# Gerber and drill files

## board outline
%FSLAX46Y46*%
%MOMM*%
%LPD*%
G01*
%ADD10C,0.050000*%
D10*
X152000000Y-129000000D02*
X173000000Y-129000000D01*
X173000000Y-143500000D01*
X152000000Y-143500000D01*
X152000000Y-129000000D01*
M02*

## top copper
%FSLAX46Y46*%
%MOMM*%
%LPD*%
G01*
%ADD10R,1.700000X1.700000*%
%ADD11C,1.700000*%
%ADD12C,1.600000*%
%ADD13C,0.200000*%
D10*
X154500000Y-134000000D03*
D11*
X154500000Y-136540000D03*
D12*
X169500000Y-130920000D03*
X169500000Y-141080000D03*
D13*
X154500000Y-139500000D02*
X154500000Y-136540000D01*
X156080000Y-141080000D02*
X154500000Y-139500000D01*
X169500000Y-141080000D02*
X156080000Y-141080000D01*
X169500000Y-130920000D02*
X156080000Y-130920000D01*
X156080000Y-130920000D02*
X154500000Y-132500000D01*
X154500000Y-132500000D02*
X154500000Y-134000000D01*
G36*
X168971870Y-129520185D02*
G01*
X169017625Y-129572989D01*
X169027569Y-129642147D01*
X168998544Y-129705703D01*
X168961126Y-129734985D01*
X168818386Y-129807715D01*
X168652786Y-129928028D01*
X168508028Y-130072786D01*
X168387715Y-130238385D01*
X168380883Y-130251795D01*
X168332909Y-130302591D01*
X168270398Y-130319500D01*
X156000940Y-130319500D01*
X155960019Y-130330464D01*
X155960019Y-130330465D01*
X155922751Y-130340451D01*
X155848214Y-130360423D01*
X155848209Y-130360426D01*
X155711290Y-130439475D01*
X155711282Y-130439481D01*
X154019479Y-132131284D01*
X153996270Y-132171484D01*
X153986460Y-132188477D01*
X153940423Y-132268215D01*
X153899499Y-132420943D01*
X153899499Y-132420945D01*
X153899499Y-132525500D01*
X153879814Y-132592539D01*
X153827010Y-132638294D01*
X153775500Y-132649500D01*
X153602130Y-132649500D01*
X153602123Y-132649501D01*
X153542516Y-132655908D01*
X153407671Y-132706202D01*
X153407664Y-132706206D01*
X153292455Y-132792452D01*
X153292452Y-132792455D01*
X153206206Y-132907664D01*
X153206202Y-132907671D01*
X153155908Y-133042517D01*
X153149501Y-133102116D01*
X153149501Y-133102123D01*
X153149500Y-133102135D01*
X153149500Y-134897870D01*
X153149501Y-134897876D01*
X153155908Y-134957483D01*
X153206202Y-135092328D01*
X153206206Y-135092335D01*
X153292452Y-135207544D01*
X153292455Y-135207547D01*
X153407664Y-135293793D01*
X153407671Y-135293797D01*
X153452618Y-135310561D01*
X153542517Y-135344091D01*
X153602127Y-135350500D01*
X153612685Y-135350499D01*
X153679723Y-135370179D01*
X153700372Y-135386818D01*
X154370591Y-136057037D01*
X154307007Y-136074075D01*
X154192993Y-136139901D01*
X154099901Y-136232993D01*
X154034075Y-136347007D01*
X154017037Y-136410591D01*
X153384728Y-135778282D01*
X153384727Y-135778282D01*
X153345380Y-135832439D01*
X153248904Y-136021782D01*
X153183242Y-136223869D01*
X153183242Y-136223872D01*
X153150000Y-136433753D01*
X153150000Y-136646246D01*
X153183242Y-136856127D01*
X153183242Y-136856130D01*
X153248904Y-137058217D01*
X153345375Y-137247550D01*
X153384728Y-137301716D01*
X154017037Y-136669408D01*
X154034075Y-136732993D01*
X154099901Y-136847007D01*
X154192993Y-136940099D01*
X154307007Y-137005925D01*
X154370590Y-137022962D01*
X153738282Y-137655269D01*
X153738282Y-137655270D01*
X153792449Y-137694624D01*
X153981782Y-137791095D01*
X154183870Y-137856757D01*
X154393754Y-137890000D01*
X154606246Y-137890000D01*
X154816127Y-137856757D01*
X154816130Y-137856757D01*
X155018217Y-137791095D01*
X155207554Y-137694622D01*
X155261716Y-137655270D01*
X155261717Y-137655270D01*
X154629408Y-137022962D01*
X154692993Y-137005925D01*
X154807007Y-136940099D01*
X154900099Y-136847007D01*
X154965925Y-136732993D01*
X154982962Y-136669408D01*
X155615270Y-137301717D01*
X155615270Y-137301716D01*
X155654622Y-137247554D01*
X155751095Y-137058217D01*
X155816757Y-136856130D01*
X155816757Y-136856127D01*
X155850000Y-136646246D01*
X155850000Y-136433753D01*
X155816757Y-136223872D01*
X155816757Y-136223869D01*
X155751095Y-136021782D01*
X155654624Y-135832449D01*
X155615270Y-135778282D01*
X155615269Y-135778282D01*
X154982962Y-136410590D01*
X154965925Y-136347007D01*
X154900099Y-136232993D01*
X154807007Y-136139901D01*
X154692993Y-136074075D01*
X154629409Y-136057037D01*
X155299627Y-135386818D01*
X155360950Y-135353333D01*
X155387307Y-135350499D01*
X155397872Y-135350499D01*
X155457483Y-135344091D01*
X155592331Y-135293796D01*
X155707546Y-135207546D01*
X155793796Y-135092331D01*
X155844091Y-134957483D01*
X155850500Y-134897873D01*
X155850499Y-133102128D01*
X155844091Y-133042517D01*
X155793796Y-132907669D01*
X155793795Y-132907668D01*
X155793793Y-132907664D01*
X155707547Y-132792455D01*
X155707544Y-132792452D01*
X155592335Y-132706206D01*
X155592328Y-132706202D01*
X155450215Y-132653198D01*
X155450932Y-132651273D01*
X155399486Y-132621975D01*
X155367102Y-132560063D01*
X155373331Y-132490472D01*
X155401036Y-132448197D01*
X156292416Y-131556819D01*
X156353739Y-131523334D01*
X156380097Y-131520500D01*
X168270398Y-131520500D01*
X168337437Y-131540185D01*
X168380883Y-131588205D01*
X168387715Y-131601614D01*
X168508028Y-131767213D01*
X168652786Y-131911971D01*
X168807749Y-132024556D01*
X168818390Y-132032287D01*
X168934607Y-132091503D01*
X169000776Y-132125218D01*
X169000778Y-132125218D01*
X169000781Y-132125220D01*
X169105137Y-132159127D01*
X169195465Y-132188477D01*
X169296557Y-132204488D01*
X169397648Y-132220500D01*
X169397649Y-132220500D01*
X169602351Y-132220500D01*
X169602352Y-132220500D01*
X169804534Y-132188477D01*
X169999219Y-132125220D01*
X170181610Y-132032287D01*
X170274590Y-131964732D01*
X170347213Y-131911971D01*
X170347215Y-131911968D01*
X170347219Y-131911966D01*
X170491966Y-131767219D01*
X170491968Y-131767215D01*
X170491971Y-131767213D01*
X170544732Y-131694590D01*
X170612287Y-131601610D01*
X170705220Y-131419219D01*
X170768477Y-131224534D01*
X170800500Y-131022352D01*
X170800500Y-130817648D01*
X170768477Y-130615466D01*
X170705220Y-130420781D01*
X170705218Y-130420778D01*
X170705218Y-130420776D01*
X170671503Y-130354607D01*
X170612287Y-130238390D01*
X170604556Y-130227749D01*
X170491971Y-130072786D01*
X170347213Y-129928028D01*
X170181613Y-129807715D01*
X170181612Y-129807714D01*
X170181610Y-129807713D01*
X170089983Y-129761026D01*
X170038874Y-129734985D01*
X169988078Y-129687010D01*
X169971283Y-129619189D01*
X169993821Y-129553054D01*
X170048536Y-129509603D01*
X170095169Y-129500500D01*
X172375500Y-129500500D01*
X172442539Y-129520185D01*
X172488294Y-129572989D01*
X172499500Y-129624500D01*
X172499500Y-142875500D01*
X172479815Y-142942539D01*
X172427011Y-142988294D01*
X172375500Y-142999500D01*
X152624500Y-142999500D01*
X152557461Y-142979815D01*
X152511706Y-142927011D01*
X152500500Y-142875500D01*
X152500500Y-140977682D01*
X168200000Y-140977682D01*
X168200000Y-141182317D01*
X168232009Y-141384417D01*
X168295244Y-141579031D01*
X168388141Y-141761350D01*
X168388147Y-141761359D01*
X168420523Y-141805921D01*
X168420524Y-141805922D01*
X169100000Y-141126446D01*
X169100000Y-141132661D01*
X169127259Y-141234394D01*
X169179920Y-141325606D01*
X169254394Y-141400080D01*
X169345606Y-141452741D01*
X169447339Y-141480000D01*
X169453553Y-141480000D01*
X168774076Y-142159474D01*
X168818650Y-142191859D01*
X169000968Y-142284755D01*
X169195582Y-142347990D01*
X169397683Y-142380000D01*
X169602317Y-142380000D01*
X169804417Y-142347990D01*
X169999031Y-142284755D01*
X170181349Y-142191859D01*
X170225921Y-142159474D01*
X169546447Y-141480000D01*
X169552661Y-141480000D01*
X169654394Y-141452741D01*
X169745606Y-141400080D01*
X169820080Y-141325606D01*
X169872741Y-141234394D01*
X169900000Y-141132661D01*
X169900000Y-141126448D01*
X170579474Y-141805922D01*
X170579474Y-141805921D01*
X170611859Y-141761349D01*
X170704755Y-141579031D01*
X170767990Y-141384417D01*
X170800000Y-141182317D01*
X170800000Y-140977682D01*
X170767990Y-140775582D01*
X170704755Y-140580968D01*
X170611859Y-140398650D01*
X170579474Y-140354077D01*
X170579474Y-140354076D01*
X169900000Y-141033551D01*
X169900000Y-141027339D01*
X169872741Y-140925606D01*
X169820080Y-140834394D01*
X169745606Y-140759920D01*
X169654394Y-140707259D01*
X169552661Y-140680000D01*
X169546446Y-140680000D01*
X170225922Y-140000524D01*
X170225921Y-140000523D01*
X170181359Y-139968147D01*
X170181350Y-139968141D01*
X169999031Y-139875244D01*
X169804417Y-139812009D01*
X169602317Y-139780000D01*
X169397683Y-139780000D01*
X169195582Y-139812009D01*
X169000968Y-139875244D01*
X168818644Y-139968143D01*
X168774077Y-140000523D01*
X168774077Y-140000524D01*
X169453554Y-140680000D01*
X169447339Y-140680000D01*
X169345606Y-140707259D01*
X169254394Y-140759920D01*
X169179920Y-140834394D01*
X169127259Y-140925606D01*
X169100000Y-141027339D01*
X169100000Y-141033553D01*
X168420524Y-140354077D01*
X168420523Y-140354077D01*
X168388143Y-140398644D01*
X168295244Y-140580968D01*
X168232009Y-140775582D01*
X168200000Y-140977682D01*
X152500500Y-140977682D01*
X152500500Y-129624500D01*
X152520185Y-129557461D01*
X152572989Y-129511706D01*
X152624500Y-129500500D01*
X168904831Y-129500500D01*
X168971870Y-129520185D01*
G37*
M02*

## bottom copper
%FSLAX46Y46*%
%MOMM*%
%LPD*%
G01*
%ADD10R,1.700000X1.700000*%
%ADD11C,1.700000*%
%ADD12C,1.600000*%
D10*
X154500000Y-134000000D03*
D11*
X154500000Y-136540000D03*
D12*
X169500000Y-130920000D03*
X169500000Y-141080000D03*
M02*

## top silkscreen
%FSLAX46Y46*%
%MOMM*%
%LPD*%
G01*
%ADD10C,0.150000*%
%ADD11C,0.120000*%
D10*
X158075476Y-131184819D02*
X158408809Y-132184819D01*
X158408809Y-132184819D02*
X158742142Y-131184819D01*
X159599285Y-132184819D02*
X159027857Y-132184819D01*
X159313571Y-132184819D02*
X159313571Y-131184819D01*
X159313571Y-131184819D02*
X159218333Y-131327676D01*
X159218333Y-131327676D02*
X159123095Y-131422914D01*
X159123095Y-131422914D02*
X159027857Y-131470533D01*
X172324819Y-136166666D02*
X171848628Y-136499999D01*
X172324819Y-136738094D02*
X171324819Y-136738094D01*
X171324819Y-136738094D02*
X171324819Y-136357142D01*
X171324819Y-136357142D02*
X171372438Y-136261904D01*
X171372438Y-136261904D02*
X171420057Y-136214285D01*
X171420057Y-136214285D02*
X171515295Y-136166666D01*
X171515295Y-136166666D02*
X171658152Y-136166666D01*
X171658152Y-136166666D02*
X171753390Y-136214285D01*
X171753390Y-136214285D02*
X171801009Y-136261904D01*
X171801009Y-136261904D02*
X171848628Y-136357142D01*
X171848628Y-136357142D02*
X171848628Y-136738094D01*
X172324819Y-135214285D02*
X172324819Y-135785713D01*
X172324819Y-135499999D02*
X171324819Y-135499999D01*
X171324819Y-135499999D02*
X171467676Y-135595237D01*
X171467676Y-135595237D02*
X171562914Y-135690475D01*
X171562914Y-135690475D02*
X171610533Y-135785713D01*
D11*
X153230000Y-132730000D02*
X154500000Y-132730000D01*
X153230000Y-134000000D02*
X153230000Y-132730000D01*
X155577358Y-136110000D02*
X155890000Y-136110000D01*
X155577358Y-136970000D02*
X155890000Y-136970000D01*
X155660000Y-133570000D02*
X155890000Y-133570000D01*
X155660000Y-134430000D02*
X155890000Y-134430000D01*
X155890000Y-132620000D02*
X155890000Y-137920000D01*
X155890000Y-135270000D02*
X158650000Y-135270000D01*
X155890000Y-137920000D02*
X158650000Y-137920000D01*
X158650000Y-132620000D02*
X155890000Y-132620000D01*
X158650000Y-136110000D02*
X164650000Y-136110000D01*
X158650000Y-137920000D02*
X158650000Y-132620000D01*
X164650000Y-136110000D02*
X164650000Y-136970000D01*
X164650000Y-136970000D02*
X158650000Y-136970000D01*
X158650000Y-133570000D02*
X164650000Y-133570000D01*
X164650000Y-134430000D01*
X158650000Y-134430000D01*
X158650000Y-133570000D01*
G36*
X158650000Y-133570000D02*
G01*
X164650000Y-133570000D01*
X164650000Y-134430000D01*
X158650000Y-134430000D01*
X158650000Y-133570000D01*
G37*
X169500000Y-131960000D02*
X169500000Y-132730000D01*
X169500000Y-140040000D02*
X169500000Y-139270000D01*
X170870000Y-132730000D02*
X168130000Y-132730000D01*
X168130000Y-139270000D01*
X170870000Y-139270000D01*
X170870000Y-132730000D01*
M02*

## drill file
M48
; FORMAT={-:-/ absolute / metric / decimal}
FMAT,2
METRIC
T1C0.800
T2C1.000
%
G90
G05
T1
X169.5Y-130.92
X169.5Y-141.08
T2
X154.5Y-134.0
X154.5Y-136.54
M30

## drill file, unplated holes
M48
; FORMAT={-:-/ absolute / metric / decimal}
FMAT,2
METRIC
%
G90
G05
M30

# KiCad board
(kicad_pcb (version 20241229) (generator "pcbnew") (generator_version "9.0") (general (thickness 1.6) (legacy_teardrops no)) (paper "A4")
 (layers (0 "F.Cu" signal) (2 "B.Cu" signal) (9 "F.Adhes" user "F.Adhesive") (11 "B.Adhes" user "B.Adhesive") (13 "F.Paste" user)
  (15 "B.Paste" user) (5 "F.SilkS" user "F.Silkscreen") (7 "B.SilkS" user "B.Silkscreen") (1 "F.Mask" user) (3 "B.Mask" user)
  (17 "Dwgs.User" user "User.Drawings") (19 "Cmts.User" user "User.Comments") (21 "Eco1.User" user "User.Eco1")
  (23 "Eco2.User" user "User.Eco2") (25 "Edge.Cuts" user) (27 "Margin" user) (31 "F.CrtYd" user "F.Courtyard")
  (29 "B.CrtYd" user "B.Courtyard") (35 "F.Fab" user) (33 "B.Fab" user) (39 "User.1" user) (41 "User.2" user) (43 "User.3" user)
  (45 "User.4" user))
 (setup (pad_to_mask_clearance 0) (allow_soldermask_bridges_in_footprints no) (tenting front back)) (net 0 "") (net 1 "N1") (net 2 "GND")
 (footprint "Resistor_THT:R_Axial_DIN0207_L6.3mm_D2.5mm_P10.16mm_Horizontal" (layer "F.Cu") (at 169.5 130.92 -90)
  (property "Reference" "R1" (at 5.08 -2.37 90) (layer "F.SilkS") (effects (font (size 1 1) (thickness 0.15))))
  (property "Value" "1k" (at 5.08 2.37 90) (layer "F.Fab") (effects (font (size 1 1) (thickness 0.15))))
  (fp_line (start 1.04 0) (end 1.81 0) (stroke (width 0.12) (type solid)) (layer "F.SilkS"))
  (fp_line (start 9.12 0) (end 8.35 0) (stroke (width 0.12) (type solid)) (layer "F.SilkS"))
  (fp_rect (start 1.81 -1.37) (end 8.35 1.37) (stroke (width 0.12) (type solid)) (fill no) (layer "F.SilkS"))
  (pad "1" thru_hole circle (at 0 0 270) (size 1.6 1.6) (drill 0.8) (layers "*.Cu" "*.Mask") (remove_unused_layers no) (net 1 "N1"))
  (pad "2" thru_hole circle (at 10.16 0 270) (size 1.6 1.6) (drill 0.8) (layers "*.Cu" "*.Mask") (remove_unused_layers no) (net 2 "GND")))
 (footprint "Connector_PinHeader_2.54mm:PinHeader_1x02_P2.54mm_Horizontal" (layer "F.Cu") (at 154.5 134)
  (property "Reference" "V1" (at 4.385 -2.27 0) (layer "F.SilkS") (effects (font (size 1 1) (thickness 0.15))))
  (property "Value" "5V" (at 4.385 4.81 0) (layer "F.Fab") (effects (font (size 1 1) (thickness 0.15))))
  (fp_line (start -1.27 -1.27) (end 0 -1.27) (stroke (width 0.12) (type solid)) (layer "F.SilkS"))
  (fp_line (start -1.27 0) (end -1.27 -1.27) (stroke (width 0.12) (type solid)) (layer "F.SilkS"))
  (fp_line (start 1.077358 2.11) (end 1.39 2.11) (stroke (width 0.12) (type solid)) (layer "F.SilkS"))
  (fp_line (start 1.077358 2.97) (end 1.39 2.97) (stroke (width 0.12) (type solid)) (layer "F.SilkS"))
  (fp_line (start 1.16 -0.43) (end 1.39 -0.43) (stroke (width 0.12) (type solid)) (layer "F.SilkS"))
  (fp_line (start 1.16 0.43) (end 1.39 0.43) (stroke (width 0.12) (type solid)) (layer "F.SilkS"))
  (fp_line (start 1.39 -1.38) (end 1.39 3.92) (stroke (width 0.12) (type solid)) (layer "F.SilkS"))
  (fp_line (start 1.39 1.27) (end 4.15 1.27) (stroke (width 0.12) (type solid)) (layer "F.SilkS"))
  (fp_line (start 1.39 3.92) (end 4.15 3.92) (stroke (width 0.12) (type solid)) (layer "F.SilkS"))
  (fp_line (start 4.15 -1.38) (end 1.39 -1.38) (stroke (width 0.12) (type solid)) (layer "F.SilkS"))
  (fp_line (start 4.15 2.11) (end 10.15 2.11) (stroke (width 0.12) (type solid)) (layer "F.SilkS"))
  (fp_line (start 4.15 3.92) (end 4.15 -1.38) (stroke (width 0.12) (type solid)) (layer "F.SilkS"))
  (fp_line (start 10.15 2.11) (end 10.15 2.97) (stroke (width 0.12) (type solid)) (layer "F.SilkS"))
  (fp_line (start 10.15 2.97) (end 4.15 2.97) (stroke (width 0.12) (type solid)) (layer "F.SilkS"))
  (fp_rect (start 4.15 -0.43) (end 10.15 0.43) (stroke (width 0.12) (type solid)) (fill yes) (layer "F.SilkS"))
  (pad "1" thru_hole rect (at 0 0) (size 1.7 1.7) (drill 1) (layers "*.Cu" "*.Mask") (remove_unused_layers no) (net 1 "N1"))
  (pad "2" thru_hole circle (at 0 2.54) (size 1.7 1.7) (drill 1) (layers "*.Cu" "*.Mask") (remove_unused_layers no) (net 2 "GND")))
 (gr_rect (start 152 129) (end 173 143.5) (stroke (width 0.05) (type default)) (fill no) (layer "Edge.Cuts"))
 (segment (start 154.5 132.5) (end 154.5 134) (width 0.2) (layer "F.Cu") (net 1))
 (segment (start 156.08 130.92) (end 154.5 132.5) (width 0.2) (layer "F.Cu") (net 1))
 (segment (start 169.5 130.92) (end 156.08 130.92) (width 0.2) (layer "F.Cu") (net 1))
 (segment (start 154.5 139.5) (end 154.5 136.54) (width 0.2) (layer "F.Cu") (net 2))
 (segment (start 156.08 141.08) (end 154.5 139.5) (width 0.2) (layer "F.Cu") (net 2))
 (segment (start 169.5 141.08) (end 156.08 141.08) (width 0.2) (layer "F.Cu") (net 2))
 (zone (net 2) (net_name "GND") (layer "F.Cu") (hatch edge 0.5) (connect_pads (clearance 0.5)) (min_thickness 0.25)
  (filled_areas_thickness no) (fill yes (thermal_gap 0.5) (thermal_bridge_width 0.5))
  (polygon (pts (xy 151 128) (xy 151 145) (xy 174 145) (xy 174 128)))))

